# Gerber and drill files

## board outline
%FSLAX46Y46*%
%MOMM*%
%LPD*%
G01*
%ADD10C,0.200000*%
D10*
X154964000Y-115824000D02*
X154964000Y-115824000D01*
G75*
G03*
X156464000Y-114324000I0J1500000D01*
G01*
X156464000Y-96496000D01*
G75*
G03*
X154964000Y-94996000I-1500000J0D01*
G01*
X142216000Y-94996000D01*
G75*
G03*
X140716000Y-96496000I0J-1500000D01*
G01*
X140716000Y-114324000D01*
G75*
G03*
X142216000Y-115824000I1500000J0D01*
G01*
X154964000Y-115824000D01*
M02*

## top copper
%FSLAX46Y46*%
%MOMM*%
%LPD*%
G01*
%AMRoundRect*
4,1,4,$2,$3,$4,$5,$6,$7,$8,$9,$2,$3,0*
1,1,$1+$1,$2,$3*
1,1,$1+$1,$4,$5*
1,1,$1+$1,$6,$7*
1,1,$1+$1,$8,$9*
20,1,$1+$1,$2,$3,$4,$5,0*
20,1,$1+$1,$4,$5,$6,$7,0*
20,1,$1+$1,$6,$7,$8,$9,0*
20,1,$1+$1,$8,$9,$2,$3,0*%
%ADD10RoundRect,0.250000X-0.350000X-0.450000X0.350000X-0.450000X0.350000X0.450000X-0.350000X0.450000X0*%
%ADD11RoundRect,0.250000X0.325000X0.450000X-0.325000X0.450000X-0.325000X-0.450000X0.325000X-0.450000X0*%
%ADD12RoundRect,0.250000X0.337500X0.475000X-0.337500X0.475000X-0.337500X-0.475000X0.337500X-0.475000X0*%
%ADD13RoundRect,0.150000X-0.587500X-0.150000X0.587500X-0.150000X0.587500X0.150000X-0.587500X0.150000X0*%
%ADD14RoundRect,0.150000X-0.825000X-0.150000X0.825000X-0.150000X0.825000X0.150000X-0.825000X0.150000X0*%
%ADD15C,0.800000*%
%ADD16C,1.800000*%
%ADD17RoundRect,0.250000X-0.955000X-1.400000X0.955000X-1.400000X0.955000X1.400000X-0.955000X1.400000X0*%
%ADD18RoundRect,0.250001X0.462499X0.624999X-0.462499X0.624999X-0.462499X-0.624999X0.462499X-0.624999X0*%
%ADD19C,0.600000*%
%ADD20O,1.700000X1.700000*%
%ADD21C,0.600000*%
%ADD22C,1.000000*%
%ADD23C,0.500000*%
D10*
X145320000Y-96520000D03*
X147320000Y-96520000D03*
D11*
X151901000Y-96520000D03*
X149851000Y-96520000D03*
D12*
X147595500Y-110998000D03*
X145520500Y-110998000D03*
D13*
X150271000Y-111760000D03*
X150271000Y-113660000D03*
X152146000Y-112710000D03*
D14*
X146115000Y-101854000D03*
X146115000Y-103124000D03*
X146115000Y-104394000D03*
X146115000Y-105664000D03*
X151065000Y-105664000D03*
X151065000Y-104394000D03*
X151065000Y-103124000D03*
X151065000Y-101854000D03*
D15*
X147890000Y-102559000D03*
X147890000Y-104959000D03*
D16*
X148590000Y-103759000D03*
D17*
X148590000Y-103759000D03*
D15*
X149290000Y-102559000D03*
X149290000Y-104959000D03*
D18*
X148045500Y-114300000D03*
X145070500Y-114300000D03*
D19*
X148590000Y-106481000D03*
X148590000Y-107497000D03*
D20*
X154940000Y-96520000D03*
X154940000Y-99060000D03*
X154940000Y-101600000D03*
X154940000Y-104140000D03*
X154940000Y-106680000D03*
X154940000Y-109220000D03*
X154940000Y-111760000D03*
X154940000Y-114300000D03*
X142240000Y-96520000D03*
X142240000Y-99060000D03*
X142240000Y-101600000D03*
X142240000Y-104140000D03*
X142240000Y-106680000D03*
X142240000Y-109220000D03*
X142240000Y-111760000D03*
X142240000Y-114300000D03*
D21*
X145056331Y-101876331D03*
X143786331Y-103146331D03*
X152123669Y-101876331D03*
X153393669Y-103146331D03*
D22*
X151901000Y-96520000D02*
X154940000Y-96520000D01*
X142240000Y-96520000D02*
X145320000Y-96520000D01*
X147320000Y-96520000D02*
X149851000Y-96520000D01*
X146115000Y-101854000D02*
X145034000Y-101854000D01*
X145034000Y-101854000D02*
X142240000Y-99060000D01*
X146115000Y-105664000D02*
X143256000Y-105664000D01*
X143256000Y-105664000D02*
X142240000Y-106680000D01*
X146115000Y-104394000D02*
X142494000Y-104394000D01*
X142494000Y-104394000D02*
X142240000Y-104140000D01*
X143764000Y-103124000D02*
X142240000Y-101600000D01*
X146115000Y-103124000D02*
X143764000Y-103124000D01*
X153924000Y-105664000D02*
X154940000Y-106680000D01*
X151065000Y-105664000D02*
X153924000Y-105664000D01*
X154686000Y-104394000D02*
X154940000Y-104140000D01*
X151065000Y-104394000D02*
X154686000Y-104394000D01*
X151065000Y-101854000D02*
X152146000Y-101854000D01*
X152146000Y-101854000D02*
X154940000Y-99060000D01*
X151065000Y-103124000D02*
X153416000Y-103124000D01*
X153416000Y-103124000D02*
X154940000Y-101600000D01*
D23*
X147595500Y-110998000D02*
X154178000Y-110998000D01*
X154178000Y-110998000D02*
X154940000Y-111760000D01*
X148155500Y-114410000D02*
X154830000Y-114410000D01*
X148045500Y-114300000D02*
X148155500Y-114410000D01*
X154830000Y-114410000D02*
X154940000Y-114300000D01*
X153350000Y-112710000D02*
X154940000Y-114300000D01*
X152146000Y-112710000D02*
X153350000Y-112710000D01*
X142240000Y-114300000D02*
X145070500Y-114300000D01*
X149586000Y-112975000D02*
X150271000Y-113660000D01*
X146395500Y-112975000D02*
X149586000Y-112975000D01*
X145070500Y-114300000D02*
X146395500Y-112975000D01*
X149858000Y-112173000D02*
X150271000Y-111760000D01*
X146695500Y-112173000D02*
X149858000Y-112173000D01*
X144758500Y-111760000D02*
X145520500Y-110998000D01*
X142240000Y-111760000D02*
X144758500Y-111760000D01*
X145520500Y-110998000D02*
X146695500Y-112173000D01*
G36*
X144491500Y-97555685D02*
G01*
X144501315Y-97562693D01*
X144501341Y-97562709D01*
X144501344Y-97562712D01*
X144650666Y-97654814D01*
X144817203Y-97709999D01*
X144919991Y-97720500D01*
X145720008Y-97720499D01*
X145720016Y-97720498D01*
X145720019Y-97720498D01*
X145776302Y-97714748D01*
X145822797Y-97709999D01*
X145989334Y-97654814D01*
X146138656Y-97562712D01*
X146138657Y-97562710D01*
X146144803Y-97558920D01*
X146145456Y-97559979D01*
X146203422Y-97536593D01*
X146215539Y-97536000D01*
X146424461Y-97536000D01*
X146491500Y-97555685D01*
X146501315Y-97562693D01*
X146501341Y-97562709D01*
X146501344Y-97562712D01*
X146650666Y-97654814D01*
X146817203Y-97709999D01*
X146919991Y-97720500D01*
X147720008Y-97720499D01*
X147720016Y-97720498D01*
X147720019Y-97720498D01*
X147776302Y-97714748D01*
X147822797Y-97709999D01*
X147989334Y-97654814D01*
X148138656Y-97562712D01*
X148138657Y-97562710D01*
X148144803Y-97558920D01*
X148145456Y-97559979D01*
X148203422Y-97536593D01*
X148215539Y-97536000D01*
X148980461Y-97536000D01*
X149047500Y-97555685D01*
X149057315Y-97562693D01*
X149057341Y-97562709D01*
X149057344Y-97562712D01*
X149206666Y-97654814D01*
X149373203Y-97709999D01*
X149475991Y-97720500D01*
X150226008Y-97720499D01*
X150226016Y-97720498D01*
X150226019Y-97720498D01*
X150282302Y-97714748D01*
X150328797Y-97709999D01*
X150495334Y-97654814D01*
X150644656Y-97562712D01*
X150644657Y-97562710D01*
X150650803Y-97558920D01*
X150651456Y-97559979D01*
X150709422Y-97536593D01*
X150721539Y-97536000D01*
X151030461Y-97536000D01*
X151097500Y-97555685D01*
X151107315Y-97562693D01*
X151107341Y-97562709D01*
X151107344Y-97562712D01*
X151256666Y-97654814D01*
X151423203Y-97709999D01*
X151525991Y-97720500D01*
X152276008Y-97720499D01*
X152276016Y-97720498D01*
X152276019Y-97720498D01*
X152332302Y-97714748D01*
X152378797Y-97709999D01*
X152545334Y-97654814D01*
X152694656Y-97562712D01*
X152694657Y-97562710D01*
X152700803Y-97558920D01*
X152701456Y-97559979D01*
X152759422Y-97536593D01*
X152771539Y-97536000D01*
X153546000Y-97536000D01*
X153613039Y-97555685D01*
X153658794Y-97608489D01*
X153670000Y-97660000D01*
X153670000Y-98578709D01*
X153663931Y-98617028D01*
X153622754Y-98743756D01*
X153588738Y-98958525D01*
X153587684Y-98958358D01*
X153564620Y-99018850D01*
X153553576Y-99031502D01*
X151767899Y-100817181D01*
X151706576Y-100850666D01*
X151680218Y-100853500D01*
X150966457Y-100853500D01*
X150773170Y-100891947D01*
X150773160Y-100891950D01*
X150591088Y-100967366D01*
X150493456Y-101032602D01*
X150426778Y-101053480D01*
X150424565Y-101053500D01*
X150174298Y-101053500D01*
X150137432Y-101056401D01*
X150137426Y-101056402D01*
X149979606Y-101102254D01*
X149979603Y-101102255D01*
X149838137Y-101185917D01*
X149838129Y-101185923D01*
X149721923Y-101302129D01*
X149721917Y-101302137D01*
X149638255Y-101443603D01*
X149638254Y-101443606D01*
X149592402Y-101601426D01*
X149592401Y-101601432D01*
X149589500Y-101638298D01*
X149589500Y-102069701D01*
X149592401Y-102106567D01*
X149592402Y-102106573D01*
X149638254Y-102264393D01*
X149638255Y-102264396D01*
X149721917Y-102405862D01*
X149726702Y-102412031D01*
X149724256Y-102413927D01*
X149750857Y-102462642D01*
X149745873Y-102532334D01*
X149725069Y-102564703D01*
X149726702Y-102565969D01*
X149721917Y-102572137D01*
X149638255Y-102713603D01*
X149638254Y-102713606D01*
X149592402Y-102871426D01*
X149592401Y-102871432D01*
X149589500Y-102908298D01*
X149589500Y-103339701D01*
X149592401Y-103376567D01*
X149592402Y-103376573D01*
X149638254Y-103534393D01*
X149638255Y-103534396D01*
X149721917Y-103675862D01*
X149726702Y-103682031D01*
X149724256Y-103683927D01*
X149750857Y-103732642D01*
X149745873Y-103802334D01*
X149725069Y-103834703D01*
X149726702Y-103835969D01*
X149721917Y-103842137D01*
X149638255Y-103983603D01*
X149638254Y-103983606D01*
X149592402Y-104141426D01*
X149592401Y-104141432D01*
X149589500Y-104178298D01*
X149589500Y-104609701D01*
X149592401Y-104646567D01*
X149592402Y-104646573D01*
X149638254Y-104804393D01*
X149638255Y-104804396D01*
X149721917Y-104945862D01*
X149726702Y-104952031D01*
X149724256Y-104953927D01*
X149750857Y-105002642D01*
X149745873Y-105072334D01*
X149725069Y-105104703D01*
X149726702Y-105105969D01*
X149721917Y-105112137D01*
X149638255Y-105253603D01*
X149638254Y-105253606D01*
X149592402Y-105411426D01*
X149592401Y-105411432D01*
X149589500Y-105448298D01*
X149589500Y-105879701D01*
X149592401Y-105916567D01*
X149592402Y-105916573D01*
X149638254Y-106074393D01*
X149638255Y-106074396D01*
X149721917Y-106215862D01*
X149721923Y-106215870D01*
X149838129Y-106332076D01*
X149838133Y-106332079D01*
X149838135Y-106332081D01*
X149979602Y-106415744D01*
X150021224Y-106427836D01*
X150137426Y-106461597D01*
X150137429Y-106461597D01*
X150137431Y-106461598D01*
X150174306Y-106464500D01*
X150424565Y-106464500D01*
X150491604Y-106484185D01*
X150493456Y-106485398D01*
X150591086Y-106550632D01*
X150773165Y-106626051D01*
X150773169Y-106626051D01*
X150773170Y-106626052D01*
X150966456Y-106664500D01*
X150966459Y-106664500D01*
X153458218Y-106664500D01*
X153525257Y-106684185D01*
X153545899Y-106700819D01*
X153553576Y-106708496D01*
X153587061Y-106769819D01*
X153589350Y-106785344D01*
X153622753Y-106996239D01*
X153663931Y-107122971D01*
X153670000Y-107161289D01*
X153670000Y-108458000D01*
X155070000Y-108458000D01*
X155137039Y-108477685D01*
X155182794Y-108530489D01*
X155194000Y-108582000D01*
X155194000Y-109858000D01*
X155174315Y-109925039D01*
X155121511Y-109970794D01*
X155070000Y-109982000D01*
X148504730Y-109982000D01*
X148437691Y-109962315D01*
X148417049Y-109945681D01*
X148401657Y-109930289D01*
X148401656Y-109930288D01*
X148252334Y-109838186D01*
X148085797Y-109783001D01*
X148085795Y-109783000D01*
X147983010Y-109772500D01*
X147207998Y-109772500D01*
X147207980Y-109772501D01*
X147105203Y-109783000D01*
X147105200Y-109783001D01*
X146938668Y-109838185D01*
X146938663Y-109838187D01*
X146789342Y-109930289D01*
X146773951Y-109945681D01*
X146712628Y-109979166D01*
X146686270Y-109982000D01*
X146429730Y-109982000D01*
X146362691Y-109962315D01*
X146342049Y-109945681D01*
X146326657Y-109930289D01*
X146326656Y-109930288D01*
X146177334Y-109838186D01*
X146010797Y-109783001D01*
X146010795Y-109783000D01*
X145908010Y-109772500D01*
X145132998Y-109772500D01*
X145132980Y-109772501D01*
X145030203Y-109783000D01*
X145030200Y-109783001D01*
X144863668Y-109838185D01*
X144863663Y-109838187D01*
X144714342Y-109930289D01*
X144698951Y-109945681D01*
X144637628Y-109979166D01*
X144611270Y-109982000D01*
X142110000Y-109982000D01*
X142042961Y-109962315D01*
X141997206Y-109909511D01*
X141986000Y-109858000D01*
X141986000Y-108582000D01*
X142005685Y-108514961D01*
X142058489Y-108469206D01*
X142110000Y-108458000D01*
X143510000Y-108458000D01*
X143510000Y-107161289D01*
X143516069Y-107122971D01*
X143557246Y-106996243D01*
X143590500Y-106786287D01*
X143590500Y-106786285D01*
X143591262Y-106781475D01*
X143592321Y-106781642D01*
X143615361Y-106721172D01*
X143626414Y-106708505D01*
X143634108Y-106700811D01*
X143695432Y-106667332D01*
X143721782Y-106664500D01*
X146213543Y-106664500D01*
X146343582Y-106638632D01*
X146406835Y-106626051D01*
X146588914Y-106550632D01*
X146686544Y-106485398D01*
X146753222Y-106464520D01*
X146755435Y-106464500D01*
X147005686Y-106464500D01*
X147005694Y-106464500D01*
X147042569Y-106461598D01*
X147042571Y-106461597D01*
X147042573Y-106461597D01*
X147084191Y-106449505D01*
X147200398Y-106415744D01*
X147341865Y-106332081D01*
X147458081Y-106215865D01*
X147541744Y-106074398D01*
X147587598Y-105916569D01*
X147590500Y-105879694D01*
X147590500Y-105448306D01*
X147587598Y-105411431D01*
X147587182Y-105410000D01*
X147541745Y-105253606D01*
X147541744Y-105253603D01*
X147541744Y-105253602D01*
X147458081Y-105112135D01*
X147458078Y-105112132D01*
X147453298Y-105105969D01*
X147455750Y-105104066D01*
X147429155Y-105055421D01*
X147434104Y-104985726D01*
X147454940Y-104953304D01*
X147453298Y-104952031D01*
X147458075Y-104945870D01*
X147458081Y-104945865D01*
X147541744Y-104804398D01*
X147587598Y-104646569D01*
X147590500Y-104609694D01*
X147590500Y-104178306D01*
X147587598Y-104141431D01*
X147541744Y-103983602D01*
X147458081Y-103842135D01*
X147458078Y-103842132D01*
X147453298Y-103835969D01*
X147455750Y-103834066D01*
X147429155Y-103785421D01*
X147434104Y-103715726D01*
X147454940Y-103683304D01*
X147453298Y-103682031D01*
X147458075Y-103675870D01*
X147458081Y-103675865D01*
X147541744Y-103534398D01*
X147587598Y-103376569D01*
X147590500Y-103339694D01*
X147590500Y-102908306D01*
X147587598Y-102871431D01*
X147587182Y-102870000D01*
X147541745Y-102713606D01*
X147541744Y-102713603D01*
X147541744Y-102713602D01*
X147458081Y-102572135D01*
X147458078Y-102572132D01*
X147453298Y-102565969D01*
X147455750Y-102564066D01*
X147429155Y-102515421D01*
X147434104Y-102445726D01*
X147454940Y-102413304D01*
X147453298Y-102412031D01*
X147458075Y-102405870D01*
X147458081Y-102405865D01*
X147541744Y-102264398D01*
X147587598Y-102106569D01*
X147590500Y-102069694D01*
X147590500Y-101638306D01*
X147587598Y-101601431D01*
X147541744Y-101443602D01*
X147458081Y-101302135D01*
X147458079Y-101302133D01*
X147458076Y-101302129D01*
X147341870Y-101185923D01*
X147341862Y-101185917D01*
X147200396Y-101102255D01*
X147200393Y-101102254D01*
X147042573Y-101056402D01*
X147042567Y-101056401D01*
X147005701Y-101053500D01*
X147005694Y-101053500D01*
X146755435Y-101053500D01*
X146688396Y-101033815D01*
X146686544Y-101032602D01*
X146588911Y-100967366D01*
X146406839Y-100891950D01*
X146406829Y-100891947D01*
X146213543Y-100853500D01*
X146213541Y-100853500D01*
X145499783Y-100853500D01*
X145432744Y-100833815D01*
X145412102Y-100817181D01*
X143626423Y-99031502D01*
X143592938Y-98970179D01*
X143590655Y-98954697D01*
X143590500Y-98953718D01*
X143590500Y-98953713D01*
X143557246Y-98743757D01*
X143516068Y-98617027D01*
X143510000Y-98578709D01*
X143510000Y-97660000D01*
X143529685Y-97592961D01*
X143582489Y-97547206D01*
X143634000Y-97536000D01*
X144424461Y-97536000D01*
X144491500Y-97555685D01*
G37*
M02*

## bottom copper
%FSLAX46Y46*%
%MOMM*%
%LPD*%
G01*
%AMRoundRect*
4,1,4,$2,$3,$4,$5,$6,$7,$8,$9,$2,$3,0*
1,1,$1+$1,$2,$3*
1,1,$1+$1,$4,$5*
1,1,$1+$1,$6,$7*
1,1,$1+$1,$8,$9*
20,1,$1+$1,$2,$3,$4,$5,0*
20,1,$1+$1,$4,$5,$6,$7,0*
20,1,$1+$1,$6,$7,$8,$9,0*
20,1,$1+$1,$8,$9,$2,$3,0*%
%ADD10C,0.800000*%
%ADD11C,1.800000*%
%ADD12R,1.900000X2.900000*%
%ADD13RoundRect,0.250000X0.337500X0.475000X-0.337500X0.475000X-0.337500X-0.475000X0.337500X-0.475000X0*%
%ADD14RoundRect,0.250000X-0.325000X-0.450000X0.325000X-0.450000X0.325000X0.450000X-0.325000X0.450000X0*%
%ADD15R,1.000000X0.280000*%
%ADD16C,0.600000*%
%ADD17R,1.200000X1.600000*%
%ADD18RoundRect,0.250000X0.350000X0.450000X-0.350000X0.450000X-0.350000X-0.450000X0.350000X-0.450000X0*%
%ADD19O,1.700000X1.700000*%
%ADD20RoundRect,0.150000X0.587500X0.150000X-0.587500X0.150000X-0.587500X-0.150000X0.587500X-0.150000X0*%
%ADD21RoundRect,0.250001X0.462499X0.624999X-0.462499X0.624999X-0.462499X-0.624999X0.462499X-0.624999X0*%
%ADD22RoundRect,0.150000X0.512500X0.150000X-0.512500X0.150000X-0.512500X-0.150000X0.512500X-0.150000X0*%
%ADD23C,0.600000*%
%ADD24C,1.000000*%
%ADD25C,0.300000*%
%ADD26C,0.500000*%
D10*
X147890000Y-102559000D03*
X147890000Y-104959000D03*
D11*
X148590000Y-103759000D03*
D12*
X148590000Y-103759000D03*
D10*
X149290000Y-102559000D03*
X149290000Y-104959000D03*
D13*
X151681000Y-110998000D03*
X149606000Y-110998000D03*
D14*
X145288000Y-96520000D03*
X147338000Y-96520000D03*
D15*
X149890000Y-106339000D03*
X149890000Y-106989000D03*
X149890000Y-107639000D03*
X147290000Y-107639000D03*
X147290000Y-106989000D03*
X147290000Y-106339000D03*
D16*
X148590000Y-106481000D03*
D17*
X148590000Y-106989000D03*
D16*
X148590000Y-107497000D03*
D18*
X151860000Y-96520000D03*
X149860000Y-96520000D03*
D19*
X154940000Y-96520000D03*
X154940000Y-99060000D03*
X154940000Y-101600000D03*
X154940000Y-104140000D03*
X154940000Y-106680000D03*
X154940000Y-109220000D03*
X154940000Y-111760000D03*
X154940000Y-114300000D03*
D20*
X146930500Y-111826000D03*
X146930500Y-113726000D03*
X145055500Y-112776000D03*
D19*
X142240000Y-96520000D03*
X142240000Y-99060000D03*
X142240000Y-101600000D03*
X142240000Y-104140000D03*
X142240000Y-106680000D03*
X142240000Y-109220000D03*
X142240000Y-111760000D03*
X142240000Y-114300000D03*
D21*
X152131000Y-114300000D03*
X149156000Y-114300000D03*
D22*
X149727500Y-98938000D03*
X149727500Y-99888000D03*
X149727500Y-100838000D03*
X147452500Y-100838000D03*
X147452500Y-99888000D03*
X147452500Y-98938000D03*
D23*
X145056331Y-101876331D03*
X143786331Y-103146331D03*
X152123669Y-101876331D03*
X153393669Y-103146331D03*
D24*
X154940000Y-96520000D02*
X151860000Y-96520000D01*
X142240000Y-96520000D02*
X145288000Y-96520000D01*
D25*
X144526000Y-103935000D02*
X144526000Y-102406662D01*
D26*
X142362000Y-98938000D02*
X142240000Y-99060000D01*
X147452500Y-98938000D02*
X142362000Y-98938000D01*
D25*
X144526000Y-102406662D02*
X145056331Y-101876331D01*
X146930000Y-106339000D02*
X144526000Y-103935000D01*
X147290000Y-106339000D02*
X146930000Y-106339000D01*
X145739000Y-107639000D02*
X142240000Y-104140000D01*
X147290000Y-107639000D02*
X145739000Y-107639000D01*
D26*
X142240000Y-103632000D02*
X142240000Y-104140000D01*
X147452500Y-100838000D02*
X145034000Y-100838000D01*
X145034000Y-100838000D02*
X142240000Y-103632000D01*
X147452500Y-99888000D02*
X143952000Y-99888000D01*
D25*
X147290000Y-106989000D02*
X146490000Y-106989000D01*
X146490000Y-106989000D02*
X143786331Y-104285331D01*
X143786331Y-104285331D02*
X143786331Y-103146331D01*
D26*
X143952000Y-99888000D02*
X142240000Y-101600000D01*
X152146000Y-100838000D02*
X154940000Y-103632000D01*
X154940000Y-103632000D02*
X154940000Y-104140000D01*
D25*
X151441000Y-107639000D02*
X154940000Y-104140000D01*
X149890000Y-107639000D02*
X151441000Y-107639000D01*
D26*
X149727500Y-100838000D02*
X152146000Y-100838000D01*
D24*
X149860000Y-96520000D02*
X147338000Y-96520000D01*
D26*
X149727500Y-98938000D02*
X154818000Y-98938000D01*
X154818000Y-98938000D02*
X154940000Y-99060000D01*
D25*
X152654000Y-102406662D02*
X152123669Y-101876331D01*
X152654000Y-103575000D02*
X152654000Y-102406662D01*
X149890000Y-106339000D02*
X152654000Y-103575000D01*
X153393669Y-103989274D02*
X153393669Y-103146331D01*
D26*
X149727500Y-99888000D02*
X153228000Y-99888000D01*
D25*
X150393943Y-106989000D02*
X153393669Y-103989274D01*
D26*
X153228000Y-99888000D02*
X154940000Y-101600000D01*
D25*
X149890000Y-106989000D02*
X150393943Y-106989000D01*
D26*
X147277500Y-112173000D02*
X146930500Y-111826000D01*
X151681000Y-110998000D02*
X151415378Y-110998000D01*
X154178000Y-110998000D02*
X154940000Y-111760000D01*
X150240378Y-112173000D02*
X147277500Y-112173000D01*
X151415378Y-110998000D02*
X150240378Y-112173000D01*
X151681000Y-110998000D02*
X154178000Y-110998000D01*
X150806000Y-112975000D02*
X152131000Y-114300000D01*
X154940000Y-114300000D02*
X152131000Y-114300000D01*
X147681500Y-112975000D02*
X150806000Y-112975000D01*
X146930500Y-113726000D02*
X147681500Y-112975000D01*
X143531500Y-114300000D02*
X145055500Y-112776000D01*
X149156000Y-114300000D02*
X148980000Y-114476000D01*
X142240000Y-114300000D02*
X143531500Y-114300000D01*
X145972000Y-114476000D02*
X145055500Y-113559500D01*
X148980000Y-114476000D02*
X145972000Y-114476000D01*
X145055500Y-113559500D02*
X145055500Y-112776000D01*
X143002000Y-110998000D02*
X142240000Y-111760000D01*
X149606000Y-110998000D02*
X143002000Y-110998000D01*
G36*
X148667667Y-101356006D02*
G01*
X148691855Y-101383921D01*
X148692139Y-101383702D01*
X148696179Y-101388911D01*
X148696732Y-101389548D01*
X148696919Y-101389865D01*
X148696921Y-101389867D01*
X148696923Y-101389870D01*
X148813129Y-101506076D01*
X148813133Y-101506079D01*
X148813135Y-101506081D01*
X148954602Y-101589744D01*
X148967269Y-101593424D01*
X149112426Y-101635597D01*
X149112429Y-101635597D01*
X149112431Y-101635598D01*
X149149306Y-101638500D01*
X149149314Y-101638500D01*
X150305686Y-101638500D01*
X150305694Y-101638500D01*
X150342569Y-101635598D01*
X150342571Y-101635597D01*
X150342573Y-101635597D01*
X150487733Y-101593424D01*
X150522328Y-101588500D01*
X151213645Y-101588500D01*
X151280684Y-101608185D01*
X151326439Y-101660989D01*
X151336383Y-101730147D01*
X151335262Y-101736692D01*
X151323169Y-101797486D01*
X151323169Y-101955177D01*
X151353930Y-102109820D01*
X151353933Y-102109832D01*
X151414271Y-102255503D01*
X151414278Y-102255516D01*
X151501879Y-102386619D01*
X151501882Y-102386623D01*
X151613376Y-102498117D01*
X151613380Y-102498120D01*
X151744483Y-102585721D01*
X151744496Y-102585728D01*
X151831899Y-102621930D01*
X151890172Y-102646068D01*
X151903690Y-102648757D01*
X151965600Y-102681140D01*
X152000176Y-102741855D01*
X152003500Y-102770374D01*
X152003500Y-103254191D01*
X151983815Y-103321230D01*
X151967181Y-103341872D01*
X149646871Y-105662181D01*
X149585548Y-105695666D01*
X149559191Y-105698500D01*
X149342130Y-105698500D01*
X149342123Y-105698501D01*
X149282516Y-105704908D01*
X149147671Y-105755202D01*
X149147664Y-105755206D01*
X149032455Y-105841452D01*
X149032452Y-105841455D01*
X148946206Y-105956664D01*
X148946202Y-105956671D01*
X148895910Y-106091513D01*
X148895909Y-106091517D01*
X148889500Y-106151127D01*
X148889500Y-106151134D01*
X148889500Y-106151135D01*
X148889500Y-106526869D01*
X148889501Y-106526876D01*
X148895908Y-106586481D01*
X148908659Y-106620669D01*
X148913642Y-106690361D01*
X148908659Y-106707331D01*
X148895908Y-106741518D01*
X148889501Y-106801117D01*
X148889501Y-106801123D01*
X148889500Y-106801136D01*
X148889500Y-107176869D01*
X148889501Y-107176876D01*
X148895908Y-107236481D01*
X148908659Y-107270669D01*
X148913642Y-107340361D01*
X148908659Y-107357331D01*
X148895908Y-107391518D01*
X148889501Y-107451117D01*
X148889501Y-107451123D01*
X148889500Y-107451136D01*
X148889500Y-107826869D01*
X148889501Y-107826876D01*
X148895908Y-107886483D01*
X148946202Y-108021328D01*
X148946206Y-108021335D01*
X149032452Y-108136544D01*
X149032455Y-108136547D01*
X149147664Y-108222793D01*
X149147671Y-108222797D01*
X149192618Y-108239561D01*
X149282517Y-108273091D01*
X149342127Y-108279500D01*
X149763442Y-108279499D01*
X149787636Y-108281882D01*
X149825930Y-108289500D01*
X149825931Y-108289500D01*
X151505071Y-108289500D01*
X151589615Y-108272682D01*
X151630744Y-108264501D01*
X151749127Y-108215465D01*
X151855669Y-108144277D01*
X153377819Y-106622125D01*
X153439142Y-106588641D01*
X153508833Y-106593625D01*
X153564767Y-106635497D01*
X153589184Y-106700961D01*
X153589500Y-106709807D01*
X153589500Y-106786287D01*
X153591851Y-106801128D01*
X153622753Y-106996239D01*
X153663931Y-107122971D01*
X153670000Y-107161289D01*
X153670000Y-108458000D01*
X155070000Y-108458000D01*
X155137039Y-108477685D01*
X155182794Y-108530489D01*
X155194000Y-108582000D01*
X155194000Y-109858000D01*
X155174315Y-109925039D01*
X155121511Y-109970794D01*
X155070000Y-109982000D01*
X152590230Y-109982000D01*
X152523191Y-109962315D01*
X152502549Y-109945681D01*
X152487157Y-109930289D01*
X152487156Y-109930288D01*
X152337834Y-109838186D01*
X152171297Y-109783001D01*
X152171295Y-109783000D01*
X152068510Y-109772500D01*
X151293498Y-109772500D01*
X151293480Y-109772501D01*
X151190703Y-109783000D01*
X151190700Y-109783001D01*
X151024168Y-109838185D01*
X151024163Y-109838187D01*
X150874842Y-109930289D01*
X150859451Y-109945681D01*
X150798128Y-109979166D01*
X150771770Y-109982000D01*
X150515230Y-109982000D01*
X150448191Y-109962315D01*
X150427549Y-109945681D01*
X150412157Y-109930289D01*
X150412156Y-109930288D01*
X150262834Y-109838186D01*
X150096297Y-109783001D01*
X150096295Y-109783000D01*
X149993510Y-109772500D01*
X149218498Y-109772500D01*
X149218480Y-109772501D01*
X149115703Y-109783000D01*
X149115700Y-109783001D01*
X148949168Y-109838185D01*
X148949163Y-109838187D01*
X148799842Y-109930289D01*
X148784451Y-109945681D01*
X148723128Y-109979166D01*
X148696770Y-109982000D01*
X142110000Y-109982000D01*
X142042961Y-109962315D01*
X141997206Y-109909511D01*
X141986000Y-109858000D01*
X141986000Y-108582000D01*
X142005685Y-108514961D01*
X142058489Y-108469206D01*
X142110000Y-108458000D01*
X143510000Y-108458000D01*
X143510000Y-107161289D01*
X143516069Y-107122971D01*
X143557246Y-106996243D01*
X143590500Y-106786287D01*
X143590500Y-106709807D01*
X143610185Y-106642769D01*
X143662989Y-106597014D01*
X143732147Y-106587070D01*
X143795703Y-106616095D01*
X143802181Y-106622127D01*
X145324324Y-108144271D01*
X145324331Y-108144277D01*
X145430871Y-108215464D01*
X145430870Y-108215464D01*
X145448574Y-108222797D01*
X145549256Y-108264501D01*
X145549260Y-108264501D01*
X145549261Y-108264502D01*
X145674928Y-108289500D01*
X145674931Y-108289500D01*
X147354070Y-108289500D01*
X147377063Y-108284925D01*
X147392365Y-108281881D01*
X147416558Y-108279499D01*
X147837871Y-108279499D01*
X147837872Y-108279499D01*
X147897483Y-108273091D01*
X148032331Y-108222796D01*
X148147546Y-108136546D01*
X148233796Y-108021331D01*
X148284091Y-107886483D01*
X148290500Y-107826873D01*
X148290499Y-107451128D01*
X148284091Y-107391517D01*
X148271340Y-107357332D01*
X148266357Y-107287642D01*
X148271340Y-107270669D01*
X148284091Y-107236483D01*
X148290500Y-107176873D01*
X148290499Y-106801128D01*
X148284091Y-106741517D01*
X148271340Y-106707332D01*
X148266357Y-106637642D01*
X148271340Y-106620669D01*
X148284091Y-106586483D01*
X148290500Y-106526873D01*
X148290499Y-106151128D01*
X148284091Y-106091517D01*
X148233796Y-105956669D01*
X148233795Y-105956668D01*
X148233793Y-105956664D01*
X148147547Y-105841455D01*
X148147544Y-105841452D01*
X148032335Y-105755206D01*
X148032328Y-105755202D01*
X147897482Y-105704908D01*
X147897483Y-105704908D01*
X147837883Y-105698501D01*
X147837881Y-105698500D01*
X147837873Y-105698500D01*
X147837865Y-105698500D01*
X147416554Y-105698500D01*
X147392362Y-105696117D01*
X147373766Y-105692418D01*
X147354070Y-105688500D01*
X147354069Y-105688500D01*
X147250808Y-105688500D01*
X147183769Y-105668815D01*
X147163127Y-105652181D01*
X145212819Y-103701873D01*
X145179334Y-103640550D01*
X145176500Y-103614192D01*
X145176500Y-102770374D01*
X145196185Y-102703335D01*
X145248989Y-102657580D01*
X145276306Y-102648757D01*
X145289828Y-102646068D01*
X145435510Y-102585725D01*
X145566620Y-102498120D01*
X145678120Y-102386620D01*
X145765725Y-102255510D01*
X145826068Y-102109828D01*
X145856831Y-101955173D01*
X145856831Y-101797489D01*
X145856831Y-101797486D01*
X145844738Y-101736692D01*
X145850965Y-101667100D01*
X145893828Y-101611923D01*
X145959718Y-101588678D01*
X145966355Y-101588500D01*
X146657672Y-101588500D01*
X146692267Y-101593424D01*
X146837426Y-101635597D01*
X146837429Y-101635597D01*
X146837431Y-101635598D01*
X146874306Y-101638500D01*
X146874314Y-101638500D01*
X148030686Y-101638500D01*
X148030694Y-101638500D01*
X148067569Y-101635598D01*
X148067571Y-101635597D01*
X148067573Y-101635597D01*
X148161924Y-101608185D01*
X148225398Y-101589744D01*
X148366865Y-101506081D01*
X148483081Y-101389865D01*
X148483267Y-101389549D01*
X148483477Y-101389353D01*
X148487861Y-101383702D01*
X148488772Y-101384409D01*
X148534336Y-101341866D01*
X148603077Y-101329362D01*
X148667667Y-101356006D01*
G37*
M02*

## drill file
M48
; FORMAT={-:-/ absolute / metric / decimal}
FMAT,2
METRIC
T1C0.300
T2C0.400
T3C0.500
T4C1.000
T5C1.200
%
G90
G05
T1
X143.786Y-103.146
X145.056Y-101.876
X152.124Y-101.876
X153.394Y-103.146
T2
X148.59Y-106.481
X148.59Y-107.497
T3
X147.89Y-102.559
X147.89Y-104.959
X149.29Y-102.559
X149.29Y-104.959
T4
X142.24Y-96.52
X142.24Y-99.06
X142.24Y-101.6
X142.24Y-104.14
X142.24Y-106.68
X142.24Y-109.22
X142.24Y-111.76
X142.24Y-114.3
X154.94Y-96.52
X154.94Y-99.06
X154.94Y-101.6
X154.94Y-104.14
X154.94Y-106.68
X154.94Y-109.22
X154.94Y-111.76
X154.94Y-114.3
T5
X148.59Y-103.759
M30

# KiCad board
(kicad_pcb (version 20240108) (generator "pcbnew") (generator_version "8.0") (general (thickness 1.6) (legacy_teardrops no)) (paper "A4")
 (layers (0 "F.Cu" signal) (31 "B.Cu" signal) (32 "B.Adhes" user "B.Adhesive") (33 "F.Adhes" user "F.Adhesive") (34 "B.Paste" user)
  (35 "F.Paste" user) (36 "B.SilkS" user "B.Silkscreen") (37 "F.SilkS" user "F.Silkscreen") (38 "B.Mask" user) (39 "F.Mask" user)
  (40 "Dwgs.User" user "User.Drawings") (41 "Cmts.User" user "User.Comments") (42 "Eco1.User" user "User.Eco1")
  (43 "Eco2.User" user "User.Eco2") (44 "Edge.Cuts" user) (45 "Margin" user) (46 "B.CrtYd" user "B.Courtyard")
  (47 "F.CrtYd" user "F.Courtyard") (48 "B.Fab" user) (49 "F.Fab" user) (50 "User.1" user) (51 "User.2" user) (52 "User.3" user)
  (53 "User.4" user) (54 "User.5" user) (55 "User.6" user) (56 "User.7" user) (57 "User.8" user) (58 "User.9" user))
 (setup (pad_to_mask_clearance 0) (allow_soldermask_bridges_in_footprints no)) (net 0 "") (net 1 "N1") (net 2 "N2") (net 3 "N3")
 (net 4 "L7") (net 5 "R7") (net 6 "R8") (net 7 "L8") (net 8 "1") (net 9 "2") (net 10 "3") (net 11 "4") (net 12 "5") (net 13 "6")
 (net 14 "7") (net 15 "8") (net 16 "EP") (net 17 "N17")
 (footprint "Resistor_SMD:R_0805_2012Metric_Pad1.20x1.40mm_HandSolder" (layer "F.Cu") (at 146.32 96.52)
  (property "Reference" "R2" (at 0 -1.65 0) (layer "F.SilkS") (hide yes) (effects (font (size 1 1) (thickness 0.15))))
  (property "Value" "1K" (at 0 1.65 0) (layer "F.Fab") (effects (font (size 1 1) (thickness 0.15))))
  (pad "1" smd roundrect (at -1 0) (size 1.2 1.4) (layers "F.Cu" "F.Paste" "F.Mask") (roundrect_rratio 0.208333) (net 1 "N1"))
  (pad "2" smd roundrect (at 1 0) (size 1.2 1.4) (layers "F.Cu" "F.Paste" "F.Mask") (roundrect_rratio 0.208333) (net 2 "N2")))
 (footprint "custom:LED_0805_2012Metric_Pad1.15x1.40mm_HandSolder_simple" (layer "F.Cu") (at 150.876 96.52 180)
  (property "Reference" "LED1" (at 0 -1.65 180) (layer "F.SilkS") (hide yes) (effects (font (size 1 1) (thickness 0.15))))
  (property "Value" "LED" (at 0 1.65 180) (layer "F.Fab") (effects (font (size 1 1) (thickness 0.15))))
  (pad "1" smd roundrect (at -1.025 0 180) (size 1.15 1.4) (layers "F.Cu" "F.Paste" "F.Mask") (roundrect_rratio 0.217391) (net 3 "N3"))
  (pad "2" smd roundrect (at 1.025 0 180) (size 1.15 1.4) (layers "F.Cu" "F.Paste" "F.Mask") (roundrect_rratio 0.217391) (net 2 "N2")))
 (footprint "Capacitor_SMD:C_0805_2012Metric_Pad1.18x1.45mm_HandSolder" (layer "F.Cu") (at 146.558 110.998 180)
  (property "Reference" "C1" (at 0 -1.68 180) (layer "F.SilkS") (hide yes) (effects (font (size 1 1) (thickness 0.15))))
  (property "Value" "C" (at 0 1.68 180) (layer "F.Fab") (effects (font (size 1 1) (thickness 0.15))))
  (pad "1" smd roundrect (at -1.0375 0 180) (size 1.175 1.45) (layers "F.Cu" "F.Paste" "F.Mask") (roundrect_rratio 0.212766) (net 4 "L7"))
  (pad "2" smd roundrect (at 1.0375 0 180) (size 1.175 1.45) (layers "F.Cu" "F.Paste" "F.Mask") (roundrect_rratio 0.212766) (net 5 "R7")))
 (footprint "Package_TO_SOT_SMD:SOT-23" (layer "F.Cu") (at 151.2085 112.71)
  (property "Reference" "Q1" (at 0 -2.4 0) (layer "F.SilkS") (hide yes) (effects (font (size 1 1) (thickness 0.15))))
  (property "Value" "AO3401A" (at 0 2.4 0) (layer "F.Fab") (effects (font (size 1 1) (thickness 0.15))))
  (pad "1" smd roundrect (at -0.9375 -0.95) (size 1.475 0.6) (layers "F.Cu" "F.Paste" "F.Mask") (roundrect_rratio 0.25) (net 5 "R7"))
  (pad "2" smd roundrect (at -0.9375 0.95) (size 1.475 0.6) (layers "F.Cu" "F.Paste" "F.Mask") (roundrect_rratio 0.25) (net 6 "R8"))
  (pad "3" smd roundrect (at 0.9375 0) (size 1.475 0.6) (layers "F.Cu" "F.Paste" "F.Mask") (roundrect_rratio 0.25) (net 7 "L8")))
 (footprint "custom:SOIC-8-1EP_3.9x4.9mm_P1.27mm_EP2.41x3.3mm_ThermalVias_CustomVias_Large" (layer "F.Cu") (at 148.59 103.759)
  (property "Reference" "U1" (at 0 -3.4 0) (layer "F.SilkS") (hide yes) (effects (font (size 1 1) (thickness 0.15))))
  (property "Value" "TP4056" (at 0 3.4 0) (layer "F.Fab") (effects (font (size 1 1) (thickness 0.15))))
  (pad "" smd roundrect (at -0.6 -0.825) (size 1.01 1.38) (layers "F.Paste") (roundrect_rratio 0.247525))
  (pad "" smd roundrect (at -0.6 0.825) (size 1.01 1.38) (layers "F.Paste") (roundrect_rratio 0.247525))
  (pad "" smd roundrect (at 0.6 -0.825) (size 1.01 1.38) (layers "F.Paste") (roundrect_rratio 0.247525))
  (pad "" smd roundrect (at 0.6 0.825) (size 1.01 1.38) (layers "F.Paste") (roundrect_rratio 0.247525))
  (pad "1" smd roundrect (at -2.475 -1.905) (size 1.95 0.6) (layers "F.Cu" "F.Paste" "F.Mask") (roundrect_rratio 0.25) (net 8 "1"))
  (pad "2" smd roundrect (at -2.475 -0.635) (size 1.95 0.6) (layers "F.Cu" "F.Paste" "F.Mask") (roundrect_rratio 0.25) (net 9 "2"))
  (pad "3" smd roundrect (at -2.475 0.635) (size 1.95 0.6) (layers "F.Cu" "F.Paste" "F.Mask") (roundrect_rratio 0.25) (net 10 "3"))
  (pad "4" smd roundrect (at -2.475 1.905) (size 1.95 0.6) (layers "F.Cu" "F.Paste" "F.Mask") (roundrect_rratio 0.25) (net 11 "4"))
  (pad "5" smd roundrect (at 2.475 1.905) (size 1.95 0.6) (layers "F.Cu" "F.Paste" "F.Mask") (roundrect_rratio 0.25) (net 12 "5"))
  (pad "6" smd roundrect (at 2.475 0.635) (size 1.95 0.6) (layers "F.Cu" "F.Paste" "F.Mask") (roundrect_rratio 0.25) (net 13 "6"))
  (pad "7" smd roundrect (at 2.475 -0.635) (size 1.95 0.6) (layers "F.Cu" "F.Paste" "F.Mask") (roundrect_rratio 0.25) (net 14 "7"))
  (pad "8" smd roundrect (at 2.475 -1.905) (size 1.95 0.6) (layers "F.Cu" "F.Paste" "F.Mask") (roundrect_rratio 0.25) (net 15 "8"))
  (pad "9" thru_hole circle (at -0.7 -1.2) (size 0.8 0.8) (drill 0.5) (layers "*.Cu") (remove_unused_layers no) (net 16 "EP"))
  (pad "9" thru_hole circle (at -0.7 1.2) (size 0.8 0.8) (drill 0.5) (layers "*.Cu") (remove_unused_layers no) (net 16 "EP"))
  (pad "9" thru_hole circle (at 0 0) (size 1.8 1.8) (drill 1.2) (layers "*.Cu") (remove_unused_layers no) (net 16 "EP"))
  (pad "9" smd rect (at 0 0) (size 1.9 2.9) (layers "B.Cu") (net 16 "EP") (zone_connect 2))
  (pad "9" smd roundrect (at 0 0) (size 2.41 3.3) (layers "F.Cu" "F.Mask") (roundrect_rratio 0.1037344398) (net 16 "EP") (zone_connect 2))
  (pad "9" thru_hole circle (at 0.7 -1.2) (size 0.8 0.8) (drill 0.5) (layers "*.Cu") (remove_unused_layers no) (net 16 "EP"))
  (pad "9" thru_hole circle (at 0.7 1.2) (size 0.8 0.8) (drill 0.5) (layers "*.Cu") (remove_unused_layers no) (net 16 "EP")))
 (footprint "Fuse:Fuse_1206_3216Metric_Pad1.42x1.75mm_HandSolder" (layer "F.Cu") (at 146.558 114.3 180)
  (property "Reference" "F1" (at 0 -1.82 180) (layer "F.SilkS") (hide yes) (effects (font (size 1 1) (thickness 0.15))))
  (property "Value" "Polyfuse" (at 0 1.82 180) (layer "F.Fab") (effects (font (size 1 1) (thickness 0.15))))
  (pad "1" smd roundrect (at -1.4875 0 180) (size 1.425 1.75) (layers "F.Cu" "F.Paste" "F.Mask") (roundrect_rratio 0.175439) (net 7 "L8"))
  (pad "2" smd roundrect (at 1.4875 0 180) (size 1.425 1.75) (layers "F.Cu" "F.Paste" "F.Mask") (roundrect_rratio 0.175439) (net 6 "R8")))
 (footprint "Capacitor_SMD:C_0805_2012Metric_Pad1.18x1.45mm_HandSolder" (layer "B.Cu") (at 150.6435 110.998 180)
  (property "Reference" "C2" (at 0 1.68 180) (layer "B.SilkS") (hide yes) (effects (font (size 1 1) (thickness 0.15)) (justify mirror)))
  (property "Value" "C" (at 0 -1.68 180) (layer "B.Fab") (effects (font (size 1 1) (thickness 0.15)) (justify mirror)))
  (pad "1" smd roundrect (at -1.0375 0 180) (size 1.175 1.45) (layers "B.Cu" "B.Paste" "B.Mask") (roundrect_rratio 0.212766) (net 4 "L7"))
  (pad "2" smd roundrect (at 1.0375 0 180) (size 1.175 1.45) (layers "B.Cu" "B.Paste" "B.Mask") (roundrect_rratio 0.212766) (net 5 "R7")))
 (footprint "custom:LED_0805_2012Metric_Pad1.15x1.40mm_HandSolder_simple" (layer "B.Cu") (at 146.313 96.52)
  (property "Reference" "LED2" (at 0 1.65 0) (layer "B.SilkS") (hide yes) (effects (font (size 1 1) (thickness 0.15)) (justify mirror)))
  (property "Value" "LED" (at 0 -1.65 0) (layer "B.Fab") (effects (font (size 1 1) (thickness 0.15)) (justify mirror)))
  (pad "1" smd roundrect (at -1.025 0) (size 1.15 1.4) (layers "B.Cu" "B.Paste" "B.Mask") (roundrect_rratio 0.217391) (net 1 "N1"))
  (pad "2" smd roundrect (at 1.025 0) (size 1.15 1.4) (layers "B.Cu" "B.Paste" "B.Mask") (roundrect_rratio 0.217391) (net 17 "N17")))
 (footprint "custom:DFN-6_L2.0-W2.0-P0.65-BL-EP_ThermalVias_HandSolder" (layer "B.Cu") (at 148.59 106.989 -90)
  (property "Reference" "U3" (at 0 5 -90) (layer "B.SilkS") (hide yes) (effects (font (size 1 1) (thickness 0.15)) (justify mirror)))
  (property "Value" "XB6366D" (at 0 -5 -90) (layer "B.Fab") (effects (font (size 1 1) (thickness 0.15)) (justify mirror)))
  (pad "1" smd rect (at -0.65 -1.3 270) (size 0.28 1) (layers "B.Cu" "B.Paste" "B.Mask") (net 15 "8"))
  (pad "2" smd rect (at 0 -1.3 270) (size 0.28 1) (layers "B.Cu" "B.Paste" "B.Mask") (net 14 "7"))
  (pad "3" smd rect (at 0.65 -1.3 270) (size 0.28 1) (layers "B.Cu" "B.Paste" "B.Mask") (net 13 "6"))
  (pad "4" smd rect (at 0.65 1.3 270) (size 0.28 1) (layers "B.Cu" "B.Paste" "B.Mask") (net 10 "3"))
  (pad "5" smd rect (at 0 1.3 270) (size 0.28 1) (layers "B.Cu" "B.Paste" "B.Mask") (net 9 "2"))
  (pad "6" smd rect (at -0.65 1.3 270) (size 0.28 1) (layers "B.Cu" "B.Paste" "B.Mask") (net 8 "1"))
  (pad "7" thru_hole circle (at -0.508 0 270) (size 0.6 0.6) (drill 0.4) (layers "*.Cu") (remove_unused_layers no) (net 16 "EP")
   (solder_mask_margin 0.148) (clearance 0.5))
  (pad "7" smd rect (at 0 0 270) (size 1.6 1.2) (layers "B.Cu" "B.Paste" "B.Mask") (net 16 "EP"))
  (pad "7" thru_hole circle (at 0.508 0 270) (size 0.6 0.6) (drill 0.4) (layers "*.Cu") (remove_unused_layers no) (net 16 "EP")
   (solder_mask_margin 0.148) (clearance 0.5)))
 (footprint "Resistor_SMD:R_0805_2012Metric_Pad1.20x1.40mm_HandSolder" (layer "B.Cu") (at 150.86 96.52 180)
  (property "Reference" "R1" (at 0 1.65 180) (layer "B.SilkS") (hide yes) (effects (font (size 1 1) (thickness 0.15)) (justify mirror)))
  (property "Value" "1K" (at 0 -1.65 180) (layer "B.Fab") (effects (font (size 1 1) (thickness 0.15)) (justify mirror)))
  (pad "1" smd roundrect (at -1 0 180) (size 1.2 1.4) (layers "B.Cu" "B.Paste" "B.Mask") (roundrect_rratio 0.208333) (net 3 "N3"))
  (pad "2" smd roundrect (at 1 0 180) (size 1.2 1.4) (layers "B.Cu" "B.Paste" "B.Mask") (roundrect_rratio 0.208333) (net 17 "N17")))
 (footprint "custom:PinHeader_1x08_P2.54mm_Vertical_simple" (layer "B.Cu") (at 154.94 96.52 180)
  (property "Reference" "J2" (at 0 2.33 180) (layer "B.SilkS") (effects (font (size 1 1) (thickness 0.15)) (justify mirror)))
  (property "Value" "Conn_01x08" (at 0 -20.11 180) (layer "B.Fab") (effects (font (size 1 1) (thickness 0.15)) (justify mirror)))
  (pad "1" thru_hole oval (at 0 0 180) (size 1.7 1.7) (drill 1) (layers "*.Cu" "*.Mask") (remove_unused_layers no) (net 3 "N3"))
  (pad "2" thru_hole oval (at 0 -2.54 180) (size 1.7 1.7) (drill 1) (layers "*.Cu" "*.Mask") (remove_unused_layers no) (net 15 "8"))
  (pad "3" thru_hole oval (at 0 -5.08 180) (size 1.7 1.7) (drill 1) (layers "*.Cu" "*.Mask") (remove_unused_layers no) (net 14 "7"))
  (pad "4" thru_hole oval (at 0 -7.62 180) (size 1.7 1.7) (drill 1) (layers "*.Cu" "*.Mask") (remove_unused_layers no) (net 13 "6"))
  (pad "5" thru_hole oval (at 0 -10.16 180) (size 1.7 1.7) (drill 1) (layers "*.Cu" "*.Mask") (remove_unused_layers no) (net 12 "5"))
  (pad "6" thru_hole oval (at 0 -12.7 180) (size 1.7 1.7) (drill 1) (layers "*.Cu" "*.Mask") (remove_unused_layers no) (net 16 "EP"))
  (pad "7" thru_hole oval (at 0 -15.24 180) (size 1.7 1.7) (drill 1) (layers "*.Cu" "*.Mask") (remove_unused_layers no) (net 4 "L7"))
  (pad "8" thru_hole oval (at 0 -17.78 180) (size 1.7 1.7) (drill 1) (layers "*.Cu" "*.Mask") (remove_unused_layers no) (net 7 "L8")))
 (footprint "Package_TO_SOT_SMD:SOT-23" (layer "B.Cu") (at 145.993 112.776 180)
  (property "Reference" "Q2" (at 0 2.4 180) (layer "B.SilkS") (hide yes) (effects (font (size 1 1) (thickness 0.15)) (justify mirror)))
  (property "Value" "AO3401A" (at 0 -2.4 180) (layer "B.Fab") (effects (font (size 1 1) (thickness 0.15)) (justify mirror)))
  (pad "1" smd roundrect (at -0.9375 0.95 180) (size 1.475 0.6) (layers "B.Cu" "B.Paste" "B.Mask") (roundrect_rratio 0.25) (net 4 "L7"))
  (pad "2" smd roundrect (at -0.9375 -0.95 180) (size 1.475 0.6) (layers "B.Cu" "B.Paste" "B.Mask") (roundrect_rratio 0.25) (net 7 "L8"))
  (pad "3" smd roundrect (at 0.9375 0 180) (size 1.475 0.6) (layers "B.Cu" "B.Paste" "B.Mask") (roundrect_rratio 0.25) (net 6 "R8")))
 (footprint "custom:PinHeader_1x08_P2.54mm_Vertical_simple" (layer "B.Cu") (at 142.24 96.52 180)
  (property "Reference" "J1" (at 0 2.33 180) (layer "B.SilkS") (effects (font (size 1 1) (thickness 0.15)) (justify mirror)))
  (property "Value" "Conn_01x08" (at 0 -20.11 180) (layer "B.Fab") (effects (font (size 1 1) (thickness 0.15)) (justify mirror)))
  (pad "1" thru_hole oval (at 0 0 180) (size 1.7 1.7) (drill 1) (layers "*.Cu" "*.Mask") (remove_unused_layers no) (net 1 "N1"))
  (pad "2" thru_hole oval (at 0 -2.54 180) (size 1.7 1.7) (drill 1) (layers "*.Cu" "*.Mask") (remove_unused_layers no) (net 8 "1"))
  (pad "3" thru_hole oval (at 0 -5.08 180) (size 1.7 1.7) (drill 1) (layers "*.Cu" "*.Mask") (remove_unused_layers no) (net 9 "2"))
  (pad "4" thru_hole oval (at 0 -7.62 180) (size 1.7 1.7) (drill 1) (layers "*.Cu" "*.Mask") (remove_unused_layers no) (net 10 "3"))
  (pad "5" thru_hole oval (at 0 -10.16 180) (size 1.7 1.7) (drill 1) (layers "*.Cu" "*.Mask") (remove_unused_layers no) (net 11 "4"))
  (pad "6" thru_hole oval (at 0 -12.7 180) (size 1.7 1.7) (drill 1) (layers "*.Cu" "*.Mask") (remove_unused_layers no) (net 16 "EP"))
  (pad "7" thru_hole oval (at 0 -15.24 180) (size 1.7 1.7) (drill 1) (layers "*.Cu" "*.Mask") (remove_unused_layers no) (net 5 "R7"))
  (pad "8" thru_hole oval (at 0 -17.78 180) (size 1.7 1.7) (drill 1) (layers "*.Cu" "*.Mask") (remove_unused_layers no) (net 6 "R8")))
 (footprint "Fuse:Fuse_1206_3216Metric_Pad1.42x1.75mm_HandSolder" (layer "B.Cu") (at 150.6435 114.3 180)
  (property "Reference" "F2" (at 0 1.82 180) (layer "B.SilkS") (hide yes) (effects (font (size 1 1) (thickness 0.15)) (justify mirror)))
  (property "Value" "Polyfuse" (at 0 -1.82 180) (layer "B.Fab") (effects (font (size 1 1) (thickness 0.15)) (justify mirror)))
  (pad "1" smd roundrect (at -1.4875 0 180) (size 1.425 1.75) (layers "B.Cu" "B.Paste" "B.Mask") (roundrect_rratio 0.175439) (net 7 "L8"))
  (pad "2" smd roundrect (at 1.4875 0 180) (size 1.425 1.75) (layers "B.Cu" "B.Paste" "B.Mask") (roundrect_rratio 0.175439) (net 6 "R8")))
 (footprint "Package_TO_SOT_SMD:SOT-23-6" (layer "B.Cu") (at 148.59 99.888 180)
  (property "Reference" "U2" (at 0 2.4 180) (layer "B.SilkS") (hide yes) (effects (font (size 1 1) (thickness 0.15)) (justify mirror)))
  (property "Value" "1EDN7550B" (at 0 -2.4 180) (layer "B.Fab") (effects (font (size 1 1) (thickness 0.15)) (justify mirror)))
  (pad "1" smd roundrect (at -1.1375 0.95 180) (size 1.325 0.6) (layers "B.Cu" "B.Paste" "B.Mask") (roundrect_rratio 0.25) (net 15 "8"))
  (pad "2" smd roundrect (at -1.1375 0 180) (size 1.325 0.6) (layers "B.Cu" "B.Paste" "B.Mask") (roundrect_rratio 0.25) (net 14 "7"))
  (pad "3" smd roundrect (at -1.1375 -0.95 180) (size 1.325 0.6) (layers "B.Cu" "B.Paste" "B.Mask") (roundrect_rratio 0.25) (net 13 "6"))
  (pad "4" smd roundrect (at 1.1375 -0.95 180) (size 1.325 0.6) (layers "B.Cu" "B.Paste" "B.Mask") (roundrect_rratio 0.25) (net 10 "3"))
  (pad "5" smd roundrect (at 1.1375 0 180) (size 1.325 0.6) (layers "B.Cu" "B.Paste" "B.Mask") (roundrect_rratio 0.25) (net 9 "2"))
  (pad "6" smd roundrect (at 1.1375 0.95 180) (size 1.325 0.6) (layers "B.Cu" "B.Paste" "B.Mask") (roundrect_rratio 0.25) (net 8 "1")))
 (gr_poly
  (pts
   (arc (start 154.964 115.824) (mid 156.02466 115.38466) (end 156.464 114.324))
   (arc (start 156.464 96.496) (mid 156.02466 95.43534) (end 154.964 94.996))
   (arc (start 142.216 94.996) (mid 141.15534 95.43534) (end 140.716 96.496))
   (arc (start 140.716 114.324) (mid 141.15534 115.38466) (end 142.216 115.824)))
  (stroke (width 0.2) (type solid)) (fill none) (layer "Edge.Cuts"))
 (segment (start 151.901 96.52) (end 154.94 96.52) (width 1) (layer "F.Cu") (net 3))
 (segment (start 154.94 96.52) (end 151.86 96.52) (width 1) (layer "B.Cu") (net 3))
 (segment (start 142.24 96.52) (end 145.32 96.52) (width 1) (layer "F.Cu") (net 1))
 (segment (start 142.24 96.52) (end 145.288 96.52) (width 1) (layer "B.Cu") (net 1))
 (segment (start 147.32 96.52) (end 149.851 96.52) (width 1) (layer "F.Cu") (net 2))
 (segment (start 146.115 101.854) (end 145.034 101.854) (width 1) (layer "F.Cu") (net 8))
 (segment (start 145.034 101.854) (end 142.24 99.06) (width 1) (layer "F.Cu") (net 8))
 (via (at 145.056331 101.876331) (size 0.6) (drill 0.3) (layers "F.Cu" "B.Cu") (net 8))
 (segment (start 144.526 103.935) (end 144.526 102.406662) (width 0.3) (layer "B.Cu") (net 8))
 (segment (start 142.362 98.938) (end 142.24 99.06) (width 0.5) (layer "B.Cu") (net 8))
 (segment (start 147.4525 98.938) (end 142.362 98.938) (width 0.5) (layer "B.Cu") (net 8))
 (segment (start 144.526 102.406662) (end 145.056331 101.876331) (width 0.3) (layer "B.Cu") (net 8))
 (segment (start 146.93 106.339) (end 144.526 103.935) (width 0.3) (layer "B.Cu") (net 8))
 (segment (start 147.29 106.339) (end 146.93 106.339) (width 0.3) (layer "B.Cu") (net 8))
 (segment (start 146.115 105.664) (end 143.256 105.664) (width 1) (layer "F.Cu") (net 11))
 (segment (start 143.256 105.664) (end 142.24 106.68) (width 1) (layer "F.Cu") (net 11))
 (segment (start 146.115 104.394) (end 142.494 104.394) (width 1) (layer "F.Cu") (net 10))
 (segment (start 142.494 104.394) (end 142.24 104.14) (width 1) (layer "F.Cu") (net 10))
 (segment (start 145.739 107.639) (end 142.24 104.14) (width 0.3) (layer "B.Cu") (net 10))
 (segment (start 147.29 107.639) (end 145.739 107.639) (width 0.3) (layer "B.Cu") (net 10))
 (segment (start 142.24 103.632) (end 142.24 104.14) (width 0.5) (layer "B.Cu") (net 10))
 (segment (start 147.4525 100.838) (end 145.034 100.838) (width 0.5) (layer "B.Cu") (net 10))
 (segment (start 145.034 100.838) (end 142.24 103.632) (width 0.5) (layer "B.Cu") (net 10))
 (segment (start 143.764 103.124) (end 142.24 101.6) (width 1) (layer "F.Cu") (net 9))
 (segment (start 146.115 103.124) (end 143.764 103.124) (width 1) (layer "F.Cu") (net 9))
 (via (at 143.786331 103.146331) (size 0.6) (drill 0.3) (layers "F.Cu" "B.Cu") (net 9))
 (segment (start 147.4525 99.888) (end 143.952 99.888) (width 0.5) (layer "B.Cu") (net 9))
 (segment (start 147.29 106.989) (end 146.49 106.989) (width 0.3) (layer "B.Cu") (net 9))
 (segment (start 146.49 106.989) (end 143.786331 104.285331) (width 0.3) (layer "B.Cu") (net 9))
 (segment (start 143.786331 104.285331) (end 143.786331 103.146331) (width 0.3) (layer "B.Cu") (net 9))
 (segment (start 143.952 99.888) (end 142.24 101.6) (width 0.5) (layer "B.Cu") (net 9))
 (segment (start 153.924 105.664) (end 154.94 106.68) (width 1) (layer "F.Cu") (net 12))
 (segment (start 151.065 105.664) (end 153.924 105.664) (width 1) (layer "F.Cu") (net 12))
 (segment (start 154.686 104.394) (end 154.94 104.14) (width 1) (layer "F.Cu") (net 13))
 (segment (start 151.065 104.394) (end 154.686 104.394) (width 1) (layer "F.Cu") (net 13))
 (segment (start 152.146 100.838) (end 154.94 103.632) (width 0.5) (layer "B.Cu") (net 13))
 (segment (start 154.94 103.632) (end 154.94 104.14) (width 0.5) (layer "B.Cu") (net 13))
 (segment (start 151.441 107.639) (end 154.94 104.14) (width 0.3) (layer "B.Cu") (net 13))
 (segment (start 149.89 107.639) (end 151.441 107.639) (width 0.3) (layer "B.Cu") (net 13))
 (segment (start 149.7275 100.838) (end 152.146 100.838) (width 0.5) (layer "B.Cu") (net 13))
 (segment (start 149.86 96.52) (end 147.338 96.52) (width 1) (layer "B.Cu") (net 17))
 (segment (start 151.065 101.854) (end 152.146 101.854) (width 1) (layer "F.Cu") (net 15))
 (segment (start 152.146 101.854) (end 154.94 99.06) (width 1) (layer "F.Cu") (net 15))
 (via (at 152.123669 101.876331) (size 0.6) (drill 0.3) (layers "F.Cu" "B.Cu") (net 15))
 (segment (start 149.7275 98.938) (end 154.818 98.938) (width 0.5) (layer "B.Cu") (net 15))
 (segment (start 154.818 98.938) (end 154.94 99.06) (width 0.5) (layer "B.Cu") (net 15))
 (segment (start 152.654 102.406662) (end 152.123669 101.876331) (width 0.3) (layer "B.Cu") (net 15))
 (segment (start 152.654 103.575) (end 152.654 102.406662) (width 0.3) (layer "B.Cu") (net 15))
 (segment (start 149.89 106.339) (end 152.654 103.575) (width 0.3) (layer "B.Cu") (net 15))
 (segment (start 151.065 103.124) (end 153.416 103.124) (width 1) (layer "F.Cu") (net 14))
 (segment (start 153.416 103.124) (end 154.94 101.6) (width 1) (layer "F.Cu") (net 14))
 (via (at 153.393669 103.146331) (size 0.6) (drill 0.3) (layers "F.Cu" "B.Cu") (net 14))
 (segment (start 153.393669 103.989274) (end 153.393669 103.146331) (width 0.3) (layer "B.Cu") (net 14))
 (segment (start 149.7275 99.888) (end 153.228 99.888) (width 0.5) (layer "B.Cu") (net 14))
 (segment (start 150.393943 106.989) (end 153.393669 103.989274) (width 0.3) (layer "B.Cu") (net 14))
 (segment (start 153.228 99.888) (end 154.94 101.6) (width 0.5) (layer "B.Cu") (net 14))
 (segment (start 149.89 106.989) (end 150.393943 106.989) (width 0.3) (layer "B.Cu") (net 14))
 (segment (start 147.5955 110.998) (end 154.178 110.998) (width 0.5) (layer "F.Cu") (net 4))
 (segment (start 154.178 110.998) (end 154.94 111.76) (width 0.5) (layer "F.Cu") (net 4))
 (segment (start 147.2775 112.173) (end 146.9305 111.826) (width 0.5) (layer "B.Cu") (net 4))
 (segment (start 151.681 110.998) (end 151.415378 110.998) (width 0.5) (layer "B.Cu") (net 4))
 (segment (start 154.178 110.998) (end 154.94 111.76) (width 0.5) (layer "B.Cu") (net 4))
 (segment (start 150.240378 112.173) (end 147.2775 112.173) (width 0.5) (layer "B.Cu") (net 4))
 (segment (start 151.415378 110.998) (end 150.240378 112.173) (width 0.5) (layer "B.Cu") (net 4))
 (segment (start 151.681 110.998) (end 154.178 110.998) (width 0.5) (layer "B.Cu") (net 4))
 (segment (start 148.1555 114.41) (end 154.83 114.41) (width 0.5) (layer "F.Cu") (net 7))
 (segment (start 148.0455 114.3) (end 148.1555 114.41) (width 0.5) (layer "F.Cu") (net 7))
 (segment (start 154.83 114.41) (end 154.94 114.3) (width 0.5) (layer "F.Cu") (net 7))
 (segment (start 153.35 112.71) (end 154.94 114.3) (width 0.5) (layer "F.Cu") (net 7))
 (segment (start 152.146 112.71) (end 153.35 112.71) (width 0.5) (layer "F.Cu") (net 7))
 (segment (start 150.806 112.975) (end 152.131 114.3) (width 0.5) (layer "B.Cu") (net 7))
 (segment (start 154.94 114.3) (end 152.131 114.3) (width 0.5) (layer "B.Cu") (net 7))
 (segment (start 147.6815 112.975) (end 150.806 112.975) (width 0.5) (layer "B.Cu") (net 7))
 (segment (start 146.9305 113.726) (end 147.6815 112.975) (width 0.5) (layer "B.Cu") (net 7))
 (segment (start 142.24 114.3) (end 145.0705 114.3) (width 0.5) (layer "F.Cu") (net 6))
 (segment (start 149.586 112.975) (end 150.271 113.66) (width 0.5) (layer "F.Cu") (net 6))
 (segment (start 146.3955 112.975) (end 149.586 112.975) (width 0.5) (layer "F.Cu") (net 6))
 (segment (start 145.0705 114.3) (end 146.3955 112.975) (width 0.5) (layer "F.Cu") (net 6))
 (segment (start 143.5315 114.3) (end 145.0555 112.776) (width 0.5) (layer "B.Cu") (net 6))
 (segment (start 149.156 114.3) (end 148.98 114.476) (width 0.5) (layer "B.Cu") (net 6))
 (segment (start 142.24 114.3) (end 143.5315 114.3) (width 0.5) (layer "B.Cu") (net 6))
 (segment (start 145.972 114.476) (end 145.0555 113.5595) (width 0.5) (layer "B.Cu") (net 6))
 (segment (start 148.98 114.476) (end 145.972 114.476) (width 0.5) (layer "B.Cu") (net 6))
 (segment (start 145.0555 113.5595) (end 145.0555 112.776) (width 0.5) (layer "B.Cu") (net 6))
 (segment (start 149.858 112.173) (end 150.271 111.76) (width 0.5) (layer "F.Cu") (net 5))
 (segment (start 146.6955 112.173) (end 149.858 112.173) (width 0.5) (layer "F.Cu") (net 5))
 (segment (start 144.7585 111.76) (end 145.5205 110.998) (width 0.5) (layer "F.Cu") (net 5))
 (segment (start 142.24 111.76) (end 144.7585 111.76) (width 0.5) (layer "F.Cu") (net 5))
 (segment (start 145.5205 110.998) (end 146.6955 112.173) (width 0.5) (layer "F.Cu") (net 5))
 (segment (start 143.002 110.998) (end 142.24 111.76) (width 0.5) (layer "B.Cu") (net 5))
 (segment (start 149.606 110.998) (end 143.002 110.998) (width 0.5) (layer "B.Cu") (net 5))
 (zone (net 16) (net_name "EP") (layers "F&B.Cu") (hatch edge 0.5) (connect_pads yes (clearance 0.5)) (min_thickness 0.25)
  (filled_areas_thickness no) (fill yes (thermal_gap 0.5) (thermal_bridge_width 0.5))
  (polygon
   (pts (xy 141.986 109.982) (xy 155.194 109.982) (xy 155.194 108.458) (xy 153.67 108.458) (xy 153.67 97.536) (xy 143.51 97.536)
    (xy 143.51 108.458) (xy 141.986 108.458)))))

